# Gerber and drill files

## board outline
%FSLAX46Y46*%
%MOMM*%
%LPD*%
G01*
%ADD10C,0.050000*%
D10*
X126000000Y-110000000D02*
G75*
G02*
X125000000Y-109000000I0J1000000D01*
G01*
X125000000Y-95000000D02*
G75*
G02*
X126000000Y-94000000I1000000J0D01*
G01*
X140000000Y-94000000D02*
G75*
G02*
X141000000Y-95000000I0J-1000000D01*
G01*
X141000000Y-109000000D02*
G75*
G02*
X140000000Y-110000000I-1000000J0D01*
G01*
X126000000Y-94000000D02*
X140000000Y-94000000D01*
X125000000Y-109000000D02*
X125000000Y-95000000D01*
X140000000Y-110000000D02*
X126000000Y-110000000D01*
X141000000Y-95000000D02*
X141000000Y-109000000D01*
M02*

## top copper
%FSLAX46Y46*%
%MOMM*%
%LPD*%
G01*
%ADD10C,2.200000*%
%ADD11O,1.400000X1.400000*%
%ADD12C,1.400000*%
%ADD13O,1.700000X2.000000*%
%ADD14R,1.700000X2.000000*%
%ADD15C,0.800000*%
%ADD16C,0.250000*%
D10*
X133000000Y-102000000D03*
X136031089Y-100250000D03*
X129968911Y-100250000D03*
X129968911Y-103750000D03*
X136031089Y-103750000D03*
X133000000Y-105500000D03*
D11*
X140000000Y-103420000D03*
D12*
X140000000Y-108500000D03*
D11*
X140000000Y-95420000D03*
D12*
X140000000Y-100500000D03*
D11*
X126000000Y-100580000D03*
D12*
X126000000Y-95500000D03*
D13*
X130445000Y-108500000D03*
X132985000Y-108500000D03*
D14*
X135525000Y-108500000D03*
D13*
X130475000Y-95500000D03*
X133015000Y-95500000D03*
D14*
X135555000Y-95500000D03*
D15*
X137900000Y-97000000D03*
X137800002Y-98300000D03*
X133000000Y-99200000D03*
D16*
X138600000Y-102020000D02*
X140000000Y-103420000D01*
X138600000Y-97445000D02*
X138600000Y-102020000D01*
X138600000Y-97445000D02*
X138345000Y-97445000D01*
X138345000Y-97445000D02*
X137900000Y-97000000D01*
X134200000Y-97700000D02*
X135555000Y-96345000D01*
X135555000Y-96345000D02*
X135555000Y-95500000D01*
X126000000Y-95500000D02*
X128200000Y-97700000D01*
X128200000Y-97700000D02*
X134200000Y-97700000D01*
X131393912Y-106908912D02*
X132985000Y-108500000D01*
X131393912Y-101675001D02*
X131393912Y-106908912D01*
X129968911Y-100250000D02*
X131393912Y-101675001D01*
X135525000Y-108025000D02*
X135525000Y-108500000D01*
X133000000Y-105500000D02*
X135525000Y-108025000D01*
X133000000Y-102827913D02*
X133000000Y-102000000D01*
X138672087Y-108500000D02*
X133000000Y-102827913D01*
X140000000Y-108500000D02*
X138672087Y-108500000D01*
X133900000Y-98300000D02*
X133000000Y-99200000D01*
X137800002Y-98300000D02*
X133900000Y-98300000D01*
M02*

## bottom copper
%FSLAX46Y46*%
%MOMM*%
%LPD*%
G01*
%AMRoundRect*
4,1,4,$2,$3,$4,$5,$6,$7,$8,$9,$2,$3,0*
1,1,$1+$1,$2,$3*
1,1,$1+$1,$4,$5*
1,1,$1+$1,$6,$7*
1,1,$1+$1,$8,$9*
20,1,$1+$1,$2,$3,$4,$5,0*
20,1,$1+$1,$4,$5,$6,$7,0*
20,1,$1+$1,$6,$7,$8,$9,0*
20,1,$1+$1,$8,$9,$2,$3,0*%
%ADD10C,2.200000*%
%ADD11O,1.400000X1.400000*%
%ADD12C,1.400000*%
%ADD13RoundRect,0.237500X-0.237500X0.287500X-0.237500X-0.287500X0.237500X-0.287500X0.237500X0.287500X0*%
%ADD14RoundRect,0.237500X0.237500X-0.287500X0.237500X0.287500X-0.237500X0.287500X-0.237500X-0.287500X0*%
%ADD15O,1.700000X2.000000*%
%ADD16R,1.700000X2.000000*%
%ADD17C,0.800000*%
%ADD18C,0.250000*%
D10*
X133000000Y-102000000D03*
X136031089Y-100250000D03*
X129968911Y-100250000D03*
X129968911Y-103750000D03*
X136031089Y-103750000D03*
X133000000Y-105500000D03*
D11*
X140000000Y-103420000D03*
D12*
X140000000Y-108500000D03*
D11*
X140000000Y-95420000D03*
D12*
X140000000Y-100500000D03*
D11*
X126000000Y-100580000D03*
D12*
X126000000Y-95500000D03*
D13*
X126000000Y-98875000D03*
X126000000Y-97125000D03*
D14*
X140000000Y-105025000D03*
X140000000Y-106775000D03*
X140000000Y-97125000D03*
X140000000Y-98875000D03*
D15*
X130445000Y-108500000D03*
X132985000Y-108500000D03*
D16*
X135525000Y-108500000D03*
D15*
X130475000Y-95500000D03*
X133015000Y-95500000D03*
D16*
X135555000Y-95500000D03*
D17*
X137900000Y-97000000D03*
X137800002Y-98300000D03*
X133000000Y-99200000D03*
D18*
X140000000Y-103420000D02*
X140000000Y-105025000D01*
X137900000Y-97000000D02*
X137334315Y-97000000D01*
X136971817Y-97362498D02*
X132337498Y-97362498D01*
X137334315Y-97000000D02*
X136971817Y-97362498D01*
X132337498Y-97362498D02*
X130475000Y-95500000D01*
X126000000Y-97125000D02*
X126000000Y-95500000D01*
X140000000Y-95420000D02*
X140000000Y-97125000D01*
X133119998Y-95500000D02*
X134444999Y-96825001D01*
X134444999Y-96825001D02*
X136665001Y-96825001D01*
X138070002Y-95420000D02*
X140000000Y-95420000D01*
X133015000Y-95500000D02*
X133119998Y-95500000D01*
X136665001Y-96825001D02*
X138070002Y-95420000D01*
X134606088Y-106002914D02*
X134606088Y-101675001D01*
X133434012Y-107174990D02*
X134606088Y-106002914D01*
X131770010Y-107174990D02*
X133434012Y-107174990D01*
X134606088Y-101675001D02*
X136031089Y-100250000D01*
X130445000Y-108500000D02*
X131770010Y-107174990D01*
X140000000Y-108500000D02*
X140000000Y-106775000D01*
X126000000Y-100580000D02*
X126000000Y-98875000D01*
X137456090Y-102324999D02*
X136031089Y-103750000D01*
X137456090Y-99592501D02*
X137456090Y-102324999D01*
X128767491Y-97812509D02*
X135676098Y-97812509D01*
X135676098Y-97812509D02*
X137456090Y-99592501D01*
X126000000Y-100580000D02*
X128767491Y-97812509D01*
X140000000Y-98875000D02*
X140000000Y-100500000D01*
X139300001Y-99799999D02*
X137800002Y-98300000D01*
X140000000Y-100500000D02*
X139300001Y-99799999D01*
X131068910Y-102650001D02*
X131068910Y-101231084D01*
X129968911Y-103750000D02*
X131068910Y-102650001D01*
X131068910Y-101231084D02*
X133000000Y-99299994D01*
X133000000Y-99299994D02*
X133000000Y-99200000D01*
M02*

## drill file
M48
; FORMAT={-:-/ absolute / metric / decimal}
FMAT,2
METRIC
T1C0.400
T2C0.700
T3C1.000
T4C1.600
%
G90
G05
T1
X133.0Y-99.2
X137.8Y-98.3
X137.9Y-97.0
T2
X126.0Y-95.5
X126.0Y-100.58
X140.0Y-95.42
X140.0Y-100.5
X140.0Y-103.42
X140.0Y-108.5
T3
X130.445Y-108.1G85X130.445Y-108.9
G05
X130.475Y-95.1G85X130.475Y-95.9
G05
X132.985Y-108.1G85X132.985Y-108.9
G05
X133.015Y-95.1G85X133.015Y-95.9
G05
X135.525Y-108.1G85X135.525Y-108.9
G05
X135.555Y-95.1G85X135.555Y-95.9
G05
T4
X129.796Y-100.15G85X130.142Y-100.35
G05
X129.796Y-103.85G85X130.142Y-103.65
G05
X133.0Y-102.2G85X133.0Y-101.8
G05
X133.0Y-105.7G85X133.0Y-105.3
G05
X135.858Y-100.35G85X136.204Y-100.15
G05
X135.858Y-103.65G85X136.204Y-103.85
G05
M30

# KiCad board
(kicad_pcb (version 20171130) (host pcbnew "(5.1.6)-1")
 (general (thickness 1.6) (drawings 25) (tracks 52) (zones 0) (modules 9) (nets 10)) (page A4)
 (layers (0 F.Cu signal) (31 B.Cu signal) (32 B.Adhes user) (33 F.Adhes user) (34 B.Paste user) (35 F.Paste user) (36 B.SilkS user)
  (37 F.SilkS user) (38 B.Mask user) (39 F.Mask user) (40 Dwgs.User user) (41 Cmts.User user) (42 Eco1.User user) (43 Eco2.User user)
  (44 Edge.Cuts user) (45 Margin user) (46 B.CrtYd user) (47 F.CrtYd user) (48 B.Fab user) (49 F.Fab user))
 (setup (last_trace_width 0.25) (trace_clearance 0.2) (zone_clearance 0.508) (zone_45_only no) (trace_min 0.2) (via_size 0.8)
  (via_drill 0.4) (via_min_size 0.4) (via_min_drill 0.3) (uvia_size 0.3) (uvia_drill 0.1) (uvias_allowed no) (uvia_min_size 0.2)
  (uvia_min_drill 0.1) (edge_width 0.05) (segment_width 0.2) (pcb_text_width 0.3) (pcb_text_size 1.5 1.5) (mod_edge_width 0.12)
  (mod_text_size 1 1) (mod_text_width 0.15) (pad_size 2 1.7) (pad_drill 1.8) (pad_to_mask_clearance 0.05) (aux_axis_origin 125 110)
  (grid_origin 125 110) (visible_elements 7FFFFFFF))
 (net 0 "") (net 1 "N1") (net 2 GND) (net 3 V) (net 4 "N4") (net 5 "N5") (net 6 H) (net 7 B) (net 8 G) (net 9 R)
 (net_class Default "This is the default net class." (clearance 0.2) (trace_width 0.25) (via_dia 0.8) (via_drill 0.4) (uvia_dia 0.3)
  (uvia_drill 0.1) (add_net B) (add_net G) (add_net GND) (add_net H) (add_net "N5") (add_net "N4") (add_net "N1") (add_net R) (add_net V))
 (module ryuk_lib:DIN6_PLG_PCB (layer B.Cu) (at 133 102 180)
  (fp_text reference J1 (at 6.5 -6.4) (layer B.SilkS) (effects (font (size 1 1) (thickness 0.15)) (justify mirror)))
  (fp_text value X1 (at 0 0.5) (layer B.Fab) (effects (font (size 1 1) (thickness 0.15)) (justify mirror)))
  (pad 6 thru_hole circle (at 0 0 180) (size 2.2 2.2) (drill oval 1.6 2) (layers *.Cu *.Mask) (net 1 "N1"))
  (pad 1 thru_hole circle (at -3.031089 1.75 120) (size 2.2 2.2) (drill oval 1.6 2) (layers *.Cu *.Mask) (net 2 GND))
  (pad 5 thru_hole circle (at 3.031089 1.75 60) (size 2.2 2.2) (drill oval 1.6 2) (layers *.Cu *.Mask) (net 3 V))
  (pad 4 thru_hole circle (at 3.031089 -1.75 120) (size 2.2 2.2) (drill oval 1.6 2) (layers *.Cu *.Mask) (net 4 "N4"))
  (pad 2 thru_hole circle (at -3.031089 -1.75 60) (size 2.2 2.2) (drill oval 1.6 2) (layers *.Cu *.Mask) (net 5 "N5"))
  (pad 3 thru_hole circle (at 0 -3.5 180) (size 2.2 2.2) (drill oval 1.6 2) (layers *.Cu *.Mask) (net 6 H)))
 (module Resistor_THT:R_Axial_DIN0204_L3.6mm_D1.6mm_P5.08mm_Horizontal (layer F.Cu) (at 140 108.5 90)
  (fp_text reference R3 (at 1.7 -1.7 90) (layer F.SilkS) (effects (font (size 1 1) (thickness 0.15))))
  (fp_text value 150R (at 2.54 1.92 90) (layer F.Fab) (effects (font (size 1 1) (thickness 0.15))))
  (pad 2 thru_hole oval (at 5.08 0 90) (size 1.4 1.4) (drill 0.7) (layers *.Cu *.Mask) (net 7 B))
  (pad 1 thru_hole circle (at 0 0 90) (size 1.4 1.4) (drill 0.7) (layers *.Cu *.Mask) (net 1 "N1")))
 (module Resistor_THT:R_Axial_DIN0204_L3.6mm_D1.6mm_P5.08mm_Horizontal (layer F.Cu) (at 140 100.5 90)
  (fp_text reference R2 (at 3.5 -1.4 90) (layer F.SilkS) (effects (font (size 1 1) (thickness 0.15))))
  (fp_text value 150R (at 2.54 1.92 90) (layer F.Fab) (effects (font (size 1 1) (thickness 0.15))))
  (pad 2 thru_hole oval (at 5.08 0 90) (size 1.4 1.4) (drill 0.7) (layers *.Cu *.Mask) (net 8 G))
  (pad 1 thru_hole circle (at 0 0 90) (size 1.4 1.4) (drill 0.7) (layers *.Cu *.Mask) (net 4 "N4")))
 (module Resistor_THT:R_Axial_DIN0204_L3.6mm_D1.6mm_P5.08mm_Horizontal (layer F.Cu) (at 126 95.5 270)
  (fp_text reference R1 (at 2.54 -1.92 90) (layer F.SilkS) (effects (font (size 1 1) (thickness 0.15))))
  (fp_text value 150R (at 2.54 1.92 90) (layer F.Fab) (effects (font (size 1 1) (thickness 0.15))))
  (pad 2 thru_hole oval (at 5.08 0 270) (size 1.4 1.4) (drill 0.7) (layers *.Cu *.Mask) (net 5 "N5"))
  (pad 1 thru_hole circle (at 0 0 270) (size 1.4 1.4) (drill 0.7) (layers *.Cu *.Mask) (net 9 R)))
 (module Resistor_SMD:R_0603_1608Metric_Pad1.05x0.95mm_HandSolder (layer B.Cu) (at 126 98 270)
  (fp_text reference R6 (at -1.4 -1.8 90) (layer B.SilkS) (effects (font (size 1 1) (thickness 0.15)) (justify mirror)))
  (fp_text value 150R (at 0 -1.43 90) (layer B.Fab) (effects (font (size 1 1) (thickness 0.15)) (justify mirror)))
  (pad 2 smd roundrect (at 0.875 0 270) (size 1.05 0.95) (layers B.Cu B.Paste B.Mask) (roundrect_rratio 0.25) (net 5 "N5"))
  (pad 1 smd roundrect (at -0.875 0 270) (size 1.05 0.95) (layers B.Cu B.Paste B.Mask) (roundrect_rratio 0.25) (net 9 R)))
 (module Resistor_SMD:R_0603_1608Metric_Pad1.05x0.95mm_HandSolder (layer B.Cu) (at 140 105.9 90)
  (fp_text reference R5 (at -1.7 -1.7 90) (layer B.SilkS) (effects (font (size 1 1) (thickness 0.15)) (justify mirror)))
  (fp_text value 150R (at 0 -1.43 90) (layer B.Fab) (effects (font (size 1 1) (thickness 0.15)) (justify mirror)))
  (pad 2 smd roundrect (at 0.875 0 90) (size 1.05 0.95) (layers B.Cu B.Paste B.Mask) (roundrect_rratio 0.25) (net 7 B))
  (pad 1 smd roundrect (at -0.875 0 90) (size 1.05 0.95) (layers B.Cu B.Paste B.Mask) (roundrect_rratio 0.25) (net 1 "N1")))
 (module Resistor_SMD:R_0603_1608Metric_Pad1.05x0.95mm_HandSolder (layer B.Cu) (at 140 98 90)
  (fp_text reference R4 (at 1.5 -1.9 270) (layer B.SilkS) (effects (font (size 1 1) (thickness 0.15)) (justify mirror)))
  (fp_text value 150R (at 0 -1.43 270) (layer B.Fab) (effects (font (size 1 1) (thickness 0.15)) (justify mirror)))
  (pad 2 smd roundrect (at 0.875 0 90) (size 1.05 0.95) (layers B.Cu B.Paste B.Mask) (roundrect_rratio 0.25) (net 8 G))
  (pad 1 smd roundrect (at -0.875 0 90) (size 1.05 0.95) (layers B.Cu B.Paste B.Mask) (roundrect_rratio 0.25) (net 4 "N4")))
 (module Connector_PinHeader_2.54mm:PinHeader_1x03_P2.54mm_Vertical (layer F.Cu) (at 135.525 108.5 270)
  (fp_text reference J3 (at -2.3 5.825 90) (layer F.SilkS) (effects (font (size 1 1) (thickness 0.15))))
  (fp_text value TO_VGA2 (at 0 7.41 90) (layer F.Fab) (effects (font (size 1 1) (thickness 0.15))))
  (pad 3 thru_hole oval (at 0 5.08 270) (size 2 1.7) (drill oval 1.8 1) (layers *.Cu *.Mask) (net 2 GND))
  (pad 2 thru_hole oval (at 0 2.54 270) (size 2 1.7) (drill oval 1.8 1) (layers *.Cu *.Mask) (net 3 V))
  (pad 1 thru_hole rect (at 0 0 270) (size 2 1.7) (drill oval 1.8 1) (layers *.Cu *.Mask) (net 6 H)))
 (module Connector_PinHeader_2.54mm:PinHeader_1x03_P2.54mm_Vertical (layer F.Cu) (at 135.555 95.5 270)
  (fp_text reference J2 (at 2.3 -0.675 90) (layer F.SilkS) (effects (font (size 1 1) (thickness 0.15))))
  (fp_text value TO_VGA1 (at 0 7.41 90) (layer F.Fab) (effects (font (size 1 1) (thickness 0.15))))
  (pad 3 thru_hole oval (at 0 5.08 270) (size 2 1.7) (drill oval 1.8 1) (layers *.Cu *.Mask) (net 7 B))
  (pad 2 thru_hole oval (at 0 2.54 270) (size 2 1.7) (drill oval 1.8 1) (layers *.Cu *.Mask) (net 8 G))
  (pad 1 thru_hole rect (at 0 0 270) (size 2 1.7) (drill oval 1.8 1) (layers *.Cu *.Mask) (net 9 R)))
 (gr_arc (start 126 109) (end 125 109) (angle -90) (layer Edge.Cuts) (width 0.05))
 (gr_arc (start 126 95) (end 126 94) (angle -90) (layer Edge.Cuts) (width 0.05))
 (gr_arc (start 140 95) (end 141 95) (angle -90) (layer Edge.Cuts) (width 0.05))
 (gr_arc (start 140 109) (end 140 110) (angle -90) (layer Edge.Cuts) (width 0.05))
 (gr_line (start 126 94) (end 140 94) (layer Edge.Cuts) (width 0.05))
 (gr_line (start 125 109) (end 125 95) (layer Edge.Cuts) (width 0.05))
 (gr_line (start 140 110) (end 126 110) (layer Edge.Cuts) (width 0.05))
 (gr_line (start 141 95) (end 141 109) (layer Edge.Cuts) (width 0.05))
 (segment (start 140 103.42) (end 140 105.025) (width 0.25) (layer B.Cu) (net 7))
 (segment (start 138.6 102.02) (end 140 103.42) (width 0.25) (layer F.Cu) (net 7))
 (segment (start 138.6 97.445) (end 138.6 102.02) (width 0.25) (layer F.Cu) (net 7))
 (via (at 137.9 97) (size 0.8) (drill 0.4) (layers F.Cu B.Cu) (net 7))
 (segment (start 138.6 97.445) (end 138.345 97.445) (width 0.25) (layer F.Cu) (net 7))
 (segment (start 138.345 97.445) (end 137.9 97) (width 0.25) (layer F.Cu) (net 7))
 (segment (start 137.9 97) (end 137.334315 97) (width 0.25) (layer B.Cu) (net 7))
 (segment (start 136.971817 97.362498) (end 132.337498 97.362498) (width 0.25) (layer B.Cu) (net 7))
 (segment (start 137.334315 97) (end 136.971817 97.362498) (width 0.25) (layer B.Cu) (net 7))
 (segment (start 132.337498 97.362498) (end 130.475 95.5) (width 0.25) (layer B.Cu) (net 7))
 (segment (start 126 97.125) (end 126 95.5) (width 0.25) (layer B.Cu) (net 9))
 (segment (start 134.2 97.7) (end 135.555 96.345) (width 0.25) (layer F.Cu) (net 9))
 (segment (start 135.555 96.345) (end 135.555 95.5) (width 0.25) (layer F.Cu) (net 9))
 (segment (start 126 95.5) (end 128.2 97.7) (width 0.25) (layer F.Cu) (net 9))
 (segment (start 128.2 97.7) (end 134.2 97.7) (width 0.25) (layer F.Cu) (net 9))
 (segment (start 140 95.42) (end 140 97.125) (width 0.25) (layer B.Cu) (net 8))
 (segment (start 133.119998 95.5) (end 134.444999 96.825001) (width 0.25) (layer B.Cu) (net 8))
 (segment (start 134.444999 96.825001) (end 136.665001 96.825001) (width 0.25) (layer B.Cu) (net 8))
 (segment (start 138.070002 95.42) (end 140 95.42) (width 0.25) (layer B.Cu) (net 8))
 (segment (start 133.015 95.5) (end 133.119998 95.5) (width 0.25) (layer B.Cu) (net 8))
 (segment (start 136.665001 96.825001) (end 138.070002 95.42) (width 0.25) (layer B.Cu) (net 8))
 (segment (start 131.393912 106.908912) (end 132.985 108.5) (width 0.25) (layer F.Cu) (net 3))
 (segment (start 131.393912 101.675001) (end 131.393912 106.908912) (width 0.25) (layer F.Cu) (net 3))
 (segment (start 129.968911 100.25) (end 131.393912 101.675001) (width 0.25) (layer F.Cu) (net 3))
 (segment (start 135.525 108.025) (end 135.525 108.5) (width 0.25) (layer F.Cu) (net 6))
 (segment (start 133 105.5) (end 135.525 108.025) (width 0.25) (layer F.Cu) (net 6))
 (segment (start 134.606088 106.002914) (end 134.606088 101.675001) (width 0.25) (layer B.Cu) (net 2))
 (segment (start 133.434012 107.17499) (end 134.606088 106.002914) (width 0.25) (layer B.Cu) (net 2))
 (segment (start 131.77001 107.17499) (end 133.434012 107.17499) (width 0.25) (layer B.Cu) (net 2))
 (segment (start 134.606088 101.675001) (end 136.031089 100.25) (width 0.25) (layer B.Cu) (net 2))
 (segment (start 130.445 108.5) (end 131.77001 107.17499) (width 0.25) (layer B.Cu) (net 2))
 (segment (start 140 108.5) (end 140 106.775) (width 0.25) (layer B.Cu) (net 1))
 (segment (start 133 102.827913) (end 133 102) (width 0.25) (layer F.Cu) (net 1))
 (segment (start 138.672087 108.5) (end 133 102.827913) (width 0.25) (layer F.Cu) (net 1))
 (segment (start 140 108.5) (end 138.672087 108.5) (width 0.25) (layer F.Cu) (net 1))
 (segment (start 126 100.58) (end 126 98.875) (width 0.25) (layer B.Cu) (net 5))
 (segment (start 137.45609 102.324999) (end 136.031089 103.75) (width 0.25) (layer B.Cu) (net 5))
 (segment (start 137.45609 99.592501) (end 137.45609 102.324999) (width 0.25) (layer B.Cu) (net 5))
 (segment (start 128.767491 97.812509) (end 135.676098 97.812509) (width 0.25) (layer B.Cu) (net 5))
 (segment (start 135.676098 97.812509) (end 137.45609 99.592501) (width 0.25) (layer B.Cu) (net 5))
 (segment (start 126 100.58) (end 128.767491 97.812509) (width 0.25) (layer B.Cu) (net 5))
 (segment (start 140 98.875) (end 140 100.5) (width 0.25) (layer B.Cu) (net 4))
 (via (at 137.800002 98.3) (size 0.8) (drill 0.4) (layers F.Cu B.Cu) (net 4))
 (segment (start 139.300001 99.799999) (end 137.800002 98.3) (width 0.25) (layer B.Cu) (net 4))
 (segment (start 140 100.5) (end 139.300001 99.799999) (width 0.25) (layer B.Cu) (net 4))
 (segment (start 133.9 98.3) (end 133 99.2) (width 0.25) (layer F.Cu) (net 4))
 (segment (start 137.800002 98.3) (end 133.9 98.3) (width 0.25) (layer F.Cu) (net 4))
 (via (at 133 99.2) (size 0.8) (drill 0.4) (layers F.Cu B.Cu) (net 4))
 (segment (start 131.06891 102.650001) (end 131.06891 101.231084) (width 0.25) (layer B.Cu) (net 4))
 (segment (start 129.968911 103.75) (end 131.06891 102.650001) (width 0.25) (layer B.Cu) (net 4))
 (segment (start 131.06891 101.231084) (end 133 99.299994) (width 0.25) (layer B.Cu) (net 4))
 (segment (start 133 99.299994) (end 133 99.2) (width 0.25) (layer B.Cu) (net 4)))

